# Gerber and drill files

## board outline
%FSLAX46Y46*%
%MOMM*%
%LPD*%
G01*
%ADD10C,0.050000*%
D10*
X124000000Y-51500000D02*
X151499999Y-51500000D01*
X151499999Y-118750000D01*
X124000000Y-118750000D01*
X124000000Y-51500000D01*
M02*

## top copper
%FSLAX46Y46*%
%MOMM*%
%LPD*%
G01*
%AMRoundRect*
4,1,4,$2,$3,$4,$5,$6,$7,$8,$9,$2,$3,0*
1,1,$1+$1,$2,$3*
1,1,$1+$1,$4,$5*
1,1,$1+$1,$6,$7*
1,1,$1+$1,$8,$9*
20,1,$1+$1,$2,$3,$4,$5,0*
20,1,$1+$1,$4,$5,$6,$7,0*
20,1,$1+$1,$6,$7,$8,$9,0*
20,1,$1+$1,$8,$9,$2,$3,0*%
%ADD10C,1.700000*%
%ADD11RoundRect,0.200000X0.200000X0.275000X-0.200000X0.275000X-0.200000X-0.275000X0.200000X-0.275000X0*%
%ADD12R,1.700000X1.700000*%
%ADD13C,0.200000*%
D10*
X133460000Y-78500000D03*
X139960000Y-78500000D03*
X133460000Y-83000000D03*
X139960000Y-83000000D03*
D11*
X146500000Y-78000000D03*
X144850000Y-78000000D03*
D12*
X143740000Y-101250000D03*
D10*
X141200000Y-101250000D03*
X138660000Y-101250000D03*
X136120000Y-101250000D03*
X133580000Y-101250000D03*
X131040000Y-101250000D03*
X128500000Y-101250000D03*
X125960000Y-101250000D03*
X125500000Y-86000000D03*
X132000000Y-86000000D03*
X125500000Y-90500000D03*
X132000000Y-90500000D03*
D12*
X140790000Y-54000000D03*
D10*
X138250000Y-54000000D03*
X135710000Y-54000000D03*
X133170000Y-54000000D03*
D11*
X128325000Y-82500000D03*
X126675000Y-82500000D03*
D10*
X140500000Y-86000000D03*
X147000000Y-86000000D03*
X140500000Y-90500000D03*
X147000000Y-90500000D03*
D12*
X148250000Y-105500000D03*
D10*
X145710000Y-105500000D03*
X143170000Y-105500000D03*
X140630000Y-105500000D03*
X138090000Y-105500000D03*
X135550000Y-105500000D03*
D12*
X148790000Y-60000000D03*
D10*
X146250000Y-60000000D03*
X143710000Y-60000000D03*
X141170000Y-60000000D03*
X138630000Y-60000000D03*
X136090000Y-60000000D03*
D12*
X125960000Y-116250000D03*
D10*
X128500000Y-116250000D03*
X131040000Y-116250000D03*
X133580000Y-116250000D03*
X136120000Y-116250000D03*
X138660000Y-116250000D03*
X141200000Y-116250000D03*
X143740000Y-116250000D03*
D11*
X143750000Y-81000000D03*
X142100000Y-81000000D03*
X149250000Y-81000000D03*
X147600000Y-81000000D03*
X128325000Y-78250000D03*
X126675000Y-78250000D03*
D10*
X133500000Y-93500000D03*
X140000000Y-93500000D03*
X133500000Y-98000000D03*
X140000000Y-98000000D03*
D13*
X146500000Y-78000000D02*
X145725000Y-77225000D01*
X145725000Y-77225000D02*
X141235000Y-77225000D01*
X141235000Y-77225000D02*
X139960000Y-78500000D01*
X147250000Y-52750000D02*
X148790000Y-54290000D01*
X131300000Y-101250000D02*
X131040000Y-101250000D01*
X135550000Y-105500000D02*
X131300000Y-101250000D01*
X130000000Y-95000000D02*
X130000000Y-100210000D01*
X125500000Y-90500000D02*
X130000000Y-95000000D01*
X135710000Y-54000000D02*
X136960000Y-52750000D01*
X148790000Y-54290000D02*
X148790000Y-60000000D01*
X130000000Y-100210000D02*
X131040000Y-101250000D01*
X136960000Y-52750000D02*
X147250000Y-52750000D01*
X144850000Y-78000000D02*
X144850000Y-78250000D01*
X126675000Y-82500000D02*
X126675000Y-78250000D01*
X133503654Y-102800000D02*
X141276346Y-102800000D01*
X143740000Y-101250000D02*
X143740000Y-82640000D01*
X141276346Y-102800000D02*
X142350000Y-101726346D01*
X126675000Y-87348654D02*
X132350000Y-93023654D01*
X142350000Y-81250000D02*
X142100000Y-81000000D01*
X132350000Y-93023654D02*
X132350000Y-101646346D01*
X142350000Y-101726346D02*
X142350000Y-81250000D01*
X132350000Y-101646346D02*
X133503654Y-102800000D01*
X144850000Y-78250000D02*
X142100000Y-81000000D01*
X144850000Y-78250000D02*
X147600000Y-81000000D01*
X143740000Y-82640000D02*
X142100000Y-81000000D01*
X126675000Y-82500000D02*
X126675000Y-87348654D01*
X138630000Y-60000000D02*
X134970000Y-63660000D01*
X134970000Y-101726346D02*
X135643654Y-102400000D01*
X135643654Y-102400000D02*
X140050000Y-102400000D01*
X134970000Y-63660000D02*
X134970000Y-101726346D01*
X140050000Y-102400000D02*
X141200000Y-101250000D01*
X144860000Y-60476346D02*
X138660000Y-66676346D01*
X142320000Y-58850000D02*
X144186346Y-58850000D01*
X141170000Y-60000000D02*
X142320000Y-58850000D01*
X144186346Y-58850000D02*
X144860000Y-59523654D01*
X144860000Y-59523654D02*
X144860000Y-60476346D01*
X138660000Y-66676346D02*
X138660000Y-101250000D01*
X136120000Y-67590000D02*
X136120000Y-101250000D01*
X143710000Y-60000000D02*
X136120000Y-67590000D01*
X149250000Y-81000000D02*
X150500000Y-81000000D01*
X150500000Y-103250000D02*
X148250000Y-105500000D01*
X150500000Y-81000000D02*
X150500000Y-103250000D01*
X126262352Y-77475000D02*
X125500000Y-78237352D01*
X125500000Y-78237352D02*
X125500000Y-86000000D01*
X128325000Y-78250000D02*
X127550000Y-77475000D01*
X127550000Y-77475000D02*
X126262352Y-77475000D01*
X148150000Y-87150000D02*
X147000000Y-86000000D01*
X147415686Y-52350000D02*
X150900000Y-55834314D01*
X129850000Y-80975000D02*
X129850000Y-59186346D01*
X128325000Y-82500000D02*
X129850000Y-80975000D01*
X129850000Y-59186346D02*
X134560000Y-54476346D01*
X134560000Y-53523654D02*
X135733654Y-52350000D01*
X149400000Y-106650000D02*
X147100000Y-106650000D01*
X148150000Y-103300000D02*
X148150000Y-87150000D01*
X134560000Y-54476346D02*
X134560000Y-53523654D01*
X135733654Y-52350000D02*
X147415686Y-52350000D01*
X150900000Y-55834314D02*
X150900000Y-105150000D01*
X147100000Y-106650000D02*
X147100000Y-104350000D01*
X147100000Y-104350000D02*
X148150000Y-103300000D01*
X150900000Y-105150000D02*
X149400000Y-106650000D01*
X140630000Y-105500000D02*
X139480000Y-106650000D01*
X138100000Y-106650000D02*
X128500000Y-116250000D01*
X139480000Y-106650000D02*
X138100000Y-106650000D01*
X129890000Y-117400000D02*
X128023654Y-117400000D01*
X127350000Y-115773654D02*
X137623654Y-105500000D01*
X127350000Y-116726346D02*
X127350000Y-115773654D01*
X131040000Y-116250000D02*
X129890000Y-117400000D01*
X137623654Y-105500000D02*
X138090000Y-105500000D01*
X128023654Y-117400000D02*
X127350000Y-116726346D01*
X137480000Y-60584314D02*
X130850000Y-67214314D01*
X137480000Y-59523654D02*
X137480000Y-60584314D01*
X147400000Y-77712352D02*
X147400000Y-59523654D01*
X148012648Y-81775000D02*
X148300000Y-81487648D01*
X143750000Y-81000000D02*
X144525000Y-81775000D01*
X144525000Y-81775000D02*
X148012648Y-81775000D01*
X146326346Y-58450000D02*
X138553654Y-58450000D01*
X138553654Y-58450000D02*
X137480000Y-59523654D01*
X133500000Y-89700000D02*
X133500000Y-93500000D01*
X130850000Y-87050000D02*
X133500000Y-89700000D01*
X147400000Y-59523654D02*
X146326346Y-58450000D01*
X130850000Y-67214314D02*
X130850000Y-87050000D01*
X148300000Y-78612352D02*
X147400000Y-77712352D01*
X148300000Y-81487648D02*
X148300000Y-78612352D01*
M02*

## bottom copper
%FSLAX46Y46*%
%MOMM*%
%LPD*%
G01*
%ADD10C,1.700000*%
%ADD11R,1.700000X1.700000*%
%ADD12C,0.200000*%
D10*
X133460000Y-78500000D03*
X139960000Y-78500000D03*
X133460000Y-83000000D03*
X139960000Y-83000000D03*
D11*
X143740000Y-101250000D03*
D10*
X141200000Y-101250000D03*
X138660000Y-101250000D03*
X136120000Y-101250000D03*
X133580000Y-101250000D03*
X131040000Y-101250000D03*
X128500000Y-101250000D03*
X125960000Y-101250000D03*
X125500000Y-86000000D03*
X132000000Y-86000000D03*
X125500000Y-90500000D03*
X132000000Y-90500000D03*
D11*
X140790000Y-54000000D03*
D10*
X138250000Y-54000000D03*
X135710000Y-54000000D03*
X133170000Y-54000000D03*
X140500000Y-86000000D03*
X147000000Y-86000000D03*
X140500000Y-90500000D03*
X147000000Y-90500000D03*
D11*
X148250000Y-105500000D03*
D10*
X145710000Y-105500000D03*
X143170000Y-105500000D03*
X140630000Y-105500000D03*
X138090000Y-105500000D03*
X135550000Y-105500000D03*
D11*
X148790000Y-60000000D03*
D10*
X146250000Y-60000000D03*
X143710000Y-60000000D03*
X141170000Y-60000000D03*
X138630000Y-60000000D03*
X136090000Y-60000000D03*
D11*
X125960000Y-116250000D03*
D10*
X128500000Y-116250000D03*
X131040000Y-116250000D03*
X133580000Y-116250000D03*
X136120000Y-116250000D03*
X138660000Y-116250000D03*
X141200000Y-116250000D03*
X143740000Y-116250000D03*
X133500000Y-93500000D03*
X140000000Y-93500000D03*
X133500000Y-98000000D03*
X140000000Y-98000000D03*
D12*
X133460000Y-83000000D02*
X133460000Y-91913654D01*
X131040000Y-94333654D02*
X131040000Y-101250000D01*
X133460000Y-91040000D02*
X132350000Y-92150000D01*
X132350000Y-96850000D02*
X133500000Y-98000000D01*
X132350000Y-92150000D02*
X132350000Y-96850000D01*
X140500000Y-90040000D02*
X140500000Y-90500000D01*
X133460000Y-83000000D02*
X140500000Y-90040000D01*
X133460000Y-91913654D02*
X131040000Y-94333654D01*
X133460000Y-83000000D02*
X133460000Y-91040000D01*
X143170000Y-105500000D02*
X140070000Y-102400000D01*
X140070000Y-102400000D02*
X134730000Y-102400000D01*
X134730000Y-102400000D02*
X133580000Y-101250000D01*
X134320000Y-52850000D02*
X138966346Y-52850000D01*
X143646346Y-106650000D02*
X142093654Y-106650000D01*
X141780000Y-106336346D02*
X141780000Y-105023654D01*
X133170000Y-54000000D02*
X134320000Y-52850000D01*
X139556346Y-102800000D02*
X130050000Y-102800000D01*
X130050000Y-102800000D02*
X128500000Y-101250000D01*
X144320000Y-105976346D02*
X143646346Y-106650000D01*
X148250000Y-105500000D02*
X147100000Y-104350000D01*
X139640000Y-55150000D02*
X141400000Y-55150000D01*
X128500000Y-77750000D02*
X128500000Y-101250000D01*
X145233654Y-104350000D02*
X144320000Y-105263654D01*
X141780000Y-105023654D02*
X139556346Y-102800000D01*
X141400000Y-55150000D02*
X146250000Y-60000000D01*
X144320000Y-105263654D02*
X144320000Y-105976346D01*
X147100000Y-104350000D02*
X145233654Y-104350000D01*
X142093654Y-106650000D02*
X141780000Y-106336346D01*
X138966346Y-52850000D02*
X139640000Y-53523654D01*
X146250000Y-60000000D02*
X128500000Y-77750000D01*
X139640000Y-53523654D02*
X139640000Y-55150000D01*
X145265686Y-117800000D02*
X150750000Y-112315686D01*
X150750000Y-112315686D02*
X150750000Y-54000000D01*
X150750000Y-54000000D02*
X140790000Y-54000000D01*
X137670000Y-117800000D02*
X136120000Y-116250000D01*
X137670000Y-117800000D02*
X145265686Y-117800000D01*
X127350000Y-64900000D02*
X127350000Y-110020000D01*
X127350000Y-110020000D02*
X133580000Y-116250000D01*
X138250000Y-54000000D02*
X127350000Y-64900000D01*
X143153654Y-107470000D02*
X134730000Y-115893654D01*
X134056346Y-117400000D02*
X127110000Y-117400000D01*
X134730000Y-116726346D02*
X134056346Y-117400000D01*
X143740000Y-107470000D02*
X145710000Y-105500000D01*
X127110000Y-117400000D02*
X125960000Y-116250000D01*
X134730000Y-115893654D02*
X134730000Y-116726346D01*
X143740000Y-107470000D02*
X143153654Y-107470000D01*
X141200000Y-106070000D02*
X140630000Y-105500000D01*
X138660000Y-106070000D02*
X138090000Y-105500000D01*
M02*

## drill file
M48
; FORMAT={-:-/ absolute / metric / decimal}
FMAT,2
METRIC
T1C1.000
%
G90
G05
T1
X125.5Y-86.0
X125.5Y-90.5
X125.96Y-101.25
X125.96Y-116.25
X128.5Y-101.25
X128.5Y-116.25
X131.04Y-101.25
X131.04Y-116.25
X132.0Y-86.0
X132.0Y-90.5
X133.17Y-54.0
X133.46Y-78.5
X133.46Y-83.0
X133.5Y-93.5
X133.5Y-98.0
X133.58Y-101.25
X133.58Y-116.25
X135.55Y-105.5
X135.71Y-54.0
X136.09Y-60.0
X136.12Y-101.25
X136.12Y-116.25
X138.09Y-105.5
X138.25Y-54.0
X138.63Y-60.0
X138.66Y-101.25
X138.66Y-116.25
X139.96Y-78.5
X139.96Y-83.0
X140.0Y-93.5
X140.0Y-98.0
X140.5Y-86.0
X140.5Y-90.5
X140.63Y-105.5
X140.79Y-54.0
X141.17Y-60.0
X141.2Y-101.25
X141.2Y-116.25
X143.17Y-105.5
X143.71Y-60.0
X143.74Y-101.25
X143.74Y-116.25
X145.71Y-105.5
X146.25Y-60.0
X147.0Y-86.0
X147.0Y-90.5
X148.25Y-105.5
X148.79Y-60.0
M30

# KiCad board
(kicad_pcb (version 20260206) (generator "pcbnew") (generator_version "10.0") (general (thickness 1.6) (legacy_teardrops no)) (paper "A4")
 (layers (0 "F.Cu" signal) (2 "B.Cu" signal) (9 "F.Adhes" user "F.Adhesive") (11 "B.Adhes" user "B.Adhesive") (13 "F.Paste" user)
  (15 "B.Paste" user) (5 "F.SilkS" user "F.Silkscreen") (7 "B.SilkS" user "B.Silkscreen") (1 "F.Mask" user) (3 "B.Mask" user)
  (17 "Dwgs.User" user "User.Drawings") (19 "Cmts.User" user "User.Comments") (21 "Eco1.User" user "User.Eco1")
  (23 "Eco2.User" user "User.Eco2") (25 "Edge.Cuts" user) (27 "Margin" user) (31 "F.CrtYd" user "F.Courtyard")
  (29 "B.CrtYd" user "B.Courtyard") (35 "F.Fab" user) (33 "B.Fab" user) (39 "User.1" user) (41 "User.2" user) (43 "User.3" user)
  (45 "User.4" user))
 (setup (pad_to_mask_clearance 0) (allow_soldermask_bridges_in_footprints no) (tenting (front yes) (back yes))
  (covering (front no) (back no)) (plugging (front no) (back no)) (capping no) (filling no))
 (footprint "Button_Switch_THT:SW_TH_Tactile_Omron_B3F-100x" (layer "F.Cu") (at 133.46 78.5)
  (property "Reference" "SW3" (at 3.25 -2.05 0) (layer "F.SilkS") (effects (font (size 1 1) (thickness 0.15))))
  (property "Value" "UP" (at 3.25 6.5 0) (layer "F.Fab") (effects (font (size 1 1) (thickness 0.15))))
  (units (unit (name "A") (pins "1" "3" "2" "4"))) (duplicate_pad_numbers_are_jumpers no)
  (pad "1" thru_hole circle (at 0 0) (size 1.7 1.7) (drill 1) (layers "*.Cu" "*.Mask") (remove_unused_layers no) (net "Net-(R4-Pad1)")
   (thermal_bridge_angle 90))
  (pad "1" thru_hole circle (at 6.5 0) (size 1.7 1.7) (drill 1) (layers "*.Cu" "*.Mask") (remove_unused_layers no) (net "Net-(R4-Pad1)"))
  (pad "2" thru_hole circle (at 0 4.5) (size 1.7 1.7) (drill 1) (layers "*.Cu" "*.Mask") (remove_unused_layers no) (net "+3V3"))
  (pad "2" thru_hole circle (at 6.5 4.5) (size 1.7 1.7) (drill 1) (layers "*.Cu" "*.Mask") (remove_unused_layers no)
   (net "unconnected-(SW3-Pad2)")))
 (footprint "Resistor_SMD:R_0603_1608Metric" (layer "F.Cu") (at 145.675 78 180)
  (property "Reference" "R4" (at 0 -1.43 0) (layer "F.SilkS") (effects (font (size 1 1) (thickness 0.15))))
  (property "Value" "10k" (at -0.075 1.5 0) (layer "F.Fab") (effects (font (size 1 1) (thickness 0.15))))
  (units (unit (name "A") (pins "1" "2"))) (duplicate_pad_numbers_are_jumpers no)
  (pad "1" smd roundrect (at -0.825 0 180) (size 0.8 0.95) (layers "F.Cu" "F.Mask" "F.Paste") (roundrect_rratio 0.25) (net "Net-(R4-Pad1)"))
  (pad "2" smd roundrect (at 0.825 0 180) (size 0.8 0.95) (layers "F.Cu" "F.Mask" "F.Paste") (roundrect_rratio 0.25) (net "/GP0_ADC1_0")))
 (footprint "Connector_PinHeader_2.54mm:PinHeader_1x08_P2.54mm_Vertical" (layer "F.Cu") (at 143.74 101.25 -90)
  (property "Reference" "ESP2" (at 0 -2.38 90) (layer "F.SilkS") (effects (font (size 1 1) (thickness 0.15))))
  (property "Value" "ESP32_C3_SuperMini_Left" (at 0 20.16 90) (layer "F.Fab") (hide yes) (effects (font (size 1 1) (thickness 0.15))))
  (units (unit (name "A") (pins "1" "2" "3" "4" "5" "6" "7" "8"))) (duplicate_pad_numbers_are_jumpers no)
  (pad "1" thru_hole rect (at 0 0 270) (size 1.7 1.7) (drill 1) (layers "*.Cu" "*.Mask") (remove_unused_layers no) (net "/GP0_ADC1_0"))
  (pad "2" thru_hole circle (at 0 2.54 270) (size 1.7 1.7) (drill 1) (layers "*.Cu" "*.Mask") (remove_unused_layers no) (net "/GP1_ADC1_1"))
  (pad "3" thru_hole circle (at 0 5.08 270) (size 1.7 1.7) (drill 1) (layers "*.Cu" "*.Mask") (remove_unused_layers no) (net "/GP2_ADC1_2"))
  (pad "4" thru_hole circle (at 0 7.62 270) (size 1.7 1.7) (drill 1) (layers "*.Cu" "*.Mask") (remove_unused_layers no) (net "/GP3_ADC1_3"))
  (pad "5" thru_hole circle (at 0 10.16 270) (size 1.7 1.7) (drill 1) (layers "*.Cu" "*.Mask") (remove_unused_layers no) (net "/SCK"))
  (pad "6" thru_hole circle (at 0 12.7 270) (size 1.7 1.7) (drill 1) (layers "*.Cu" "*.Mask") (remove_unused_layers no) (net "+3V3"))
  (pad "7" thru_hole circle (at 0 15.24 270) (size 1.7 1.7) (drill 1) (layers "*.Cu" "*.Mask") (remove_unused_layers no) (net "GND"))
  (pad "8" thru_hole circle (at 0 17.78 270) (size 1.7 1.7) (drill 1) (layers "*.Cu" "*.Mask") (remove_unused_layers no)
   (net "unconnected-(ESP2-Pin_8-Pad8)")))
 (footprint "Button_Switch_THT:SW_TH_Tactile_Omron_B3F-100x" (layer "F.Cu") (at 125.5 86)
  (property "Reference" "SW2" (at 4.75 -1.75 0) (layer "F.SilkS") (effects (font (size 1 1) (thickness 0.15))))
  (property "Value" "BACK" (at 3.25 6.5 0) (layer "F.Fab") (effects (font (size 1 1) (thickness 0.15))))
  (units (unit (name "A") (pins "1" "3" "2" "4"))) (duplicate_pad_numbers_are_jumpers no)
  (pad "1" thru_hole circle (at 0 0) (size 1.7 1.7) (drill 1) (layers "*.Cu" "*.Mask") (remove_unused_layers no) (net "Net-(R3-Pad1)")
   (thermal_bridge_angle 90))
  (pad "1" thru_hole circle (at 6.5 0) (size 1.7 1.7) (drill 1) (layers "*.Cu" "*.Mask") (remove_unused_layers no) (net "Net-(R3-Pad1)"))
  (pad "2" thru_hole circle (at 0 4.5) (size 1.7 1.7) (drill 1) (layers "*.Cu" "*.Mask") (remove_unused_layers no) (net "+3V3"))
  (pad "2" thru_hole circle (at 6.5 4.5) (size 1.7 1.7) (drill 1) (layers "*.Cu" "*.Mask") (remove_unused_layers no)
   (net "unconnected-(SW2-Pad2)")))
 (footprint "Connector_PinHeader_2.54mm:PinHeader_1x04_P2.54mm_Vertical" (layer "F.Cu") (at 140.79 54 -90)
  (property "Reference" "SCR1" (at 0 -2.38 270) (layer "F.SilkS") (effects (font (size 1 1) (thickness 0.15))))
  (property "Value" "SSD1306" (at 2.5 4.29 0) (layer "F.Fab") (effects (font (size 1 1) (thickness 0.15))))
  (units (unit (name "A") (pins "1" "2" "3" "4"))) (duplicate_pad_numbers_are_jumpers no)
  (pad "1" thru_hole rect (at 0 0 270) (size 1.7 1.7) (drill 1) (layers "*.Cu" "*.Mask") (remove_unused_layers no) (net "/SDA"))
  (pad "2" thru_hole circle (at 0 2.54 270) (size 1.7 1.7) (drill 1) (layers "*.Cu" "*.Mask") (remove_unused_layers no) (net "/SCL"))
  (pad "3" thru_hole circle (at 0 5.08 270) (size 1.7 1.7) (drill 1) (layers "*.Cu" "*.Mask") (remove_unused_layers no) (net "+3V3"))
  (pad "4" thru_hole circle (at 0 7.62 270) (size 1.7 1.7) (drill 1) (layers "*.Cu" "*.Mask") (remove_unused_layers no) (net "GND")))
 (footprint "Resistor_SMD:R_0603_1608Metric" (layer "F.Cu") (at 127.5 82.5 180)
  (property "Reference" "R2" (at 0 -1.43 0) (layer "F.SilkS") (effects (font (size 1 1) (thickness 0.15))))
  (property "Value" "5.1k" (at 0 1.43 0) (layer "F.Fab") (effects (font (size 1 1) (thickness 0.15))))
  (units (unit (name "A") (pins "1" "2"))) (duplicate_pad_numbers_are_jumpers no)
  (pad "1" smd roundrect (at -0.825 0 180) (size 0.8 0.95) (layers "F.Cu" "F.Mask" "F.Paste") (roundrect_rratio 0.25) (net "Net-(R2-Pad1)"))
  (pad "2" smd roundrect (at 0.825 0 180) (size 0.8 0.95) (layers "F.Cu" "F.Mask" "F.Paste") (roundrect_rratio 0.25) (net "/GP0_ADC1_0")))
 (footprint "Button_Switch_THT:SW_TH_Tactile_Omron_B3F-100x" (layer "F.Cu") (at 140.5 86)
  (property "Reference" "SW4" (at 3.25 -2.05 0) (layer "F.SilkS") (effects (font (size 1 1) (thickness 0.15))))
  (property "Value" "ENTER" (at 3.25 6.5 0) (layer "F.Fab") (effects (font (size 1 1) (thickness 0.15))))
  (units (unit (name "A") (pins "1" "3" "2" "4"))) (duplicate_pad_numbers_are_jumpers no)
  (pad "1" thru_hole circle (at 0 0) (size 1.7 1.7) (drill 1) (layers "*.Cu" "*.Mask") (remove_unused_layers no) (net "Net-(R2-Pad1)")
   (thermal_bridge_angle 90))
  (pad "1" thru_hole circle (at 6.5 0) (size 1.7 1.7) (drill 1) (layers "*.Cu" "*.Mask") (remove_unused_layers no) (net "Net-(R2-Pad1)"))
  (pad "2" thru_hole circle (at 0 4.5) (size 1.7 1.7) (drill 1) (layers "*.Cu" "*.Mask") (remove_unused_layers no) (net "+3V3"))
  (pad "2" thru_hole circle (at 6.5 4.5) (size 1.7 1.7) (drill 1) (layers "*.Cu" "*.Mask") (remove_unused_layers no)
   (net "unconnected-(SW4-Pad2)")))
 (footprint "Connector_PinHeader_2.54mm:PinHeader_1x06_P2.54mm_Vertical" (layer "F.Cu") (at 148.25 105.5 -90)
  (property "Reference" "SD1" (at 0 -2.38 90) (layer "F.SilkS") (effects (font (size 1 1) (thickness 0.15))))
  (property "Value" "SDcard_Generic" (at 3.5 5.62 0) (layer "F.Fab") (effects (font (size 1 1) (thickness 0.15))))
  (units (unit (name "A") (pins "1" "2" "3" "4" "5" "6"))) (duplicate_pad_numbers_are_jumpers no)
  (pad "1" thru_hole rect (at 0 0 270) (size 1.7 1.7) (drill 1) (layers "*.Cu" "*.Mask") (remove_unused_layers no) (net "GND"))
  (pad "2" thru_hole circle (at 0 2.54 270) (size 1.7 1.7) (drill 1) (layers "*.Cu" "*.Mask") (remove_unused_layers no) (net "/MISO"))
  (pad "3" thru_hole circle (at 0 5.08 270) (size 1.7 1.7) (drill 1) (layers "*.Cu" "*.Mask") (remove_unused_layers no) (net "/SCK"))
  (pad "4" thru_hole circle (at 0 7.62 270) (size 1.7 1.7) (drill 1) (layers "*.Cu" "*.Mask") (remove_unused_layers no) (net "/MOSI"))
  (pad "5" thru_hole circle (at 0 10.16 270) (size 1.7 1.7) (drill 1) (layers "*.Cu" "*.Mask") (remove_unused_layers no) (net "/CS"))
  (pad "6" thru_hole circle (at 0 12.7 270) (size 1.7 1.7) (drill 1) (layers "*.Cu" "*.Mask") (remove_unused_layers no) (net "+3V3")))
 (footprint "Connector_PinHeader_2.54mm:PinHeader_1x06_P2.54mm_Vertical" (layer "F.Cu") (at 148.79 60 -90)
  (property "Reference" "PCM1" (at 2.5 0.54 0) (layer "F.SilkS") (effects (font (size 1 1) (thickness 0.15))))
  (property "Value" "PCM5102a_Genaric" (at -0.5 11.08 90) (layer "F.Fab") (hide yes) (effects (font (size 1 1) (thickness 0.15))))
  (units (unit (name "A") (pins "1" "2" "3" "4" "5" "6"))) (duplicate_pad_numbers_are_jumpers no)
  (pad "1" thru_hole rect (at 0 0 270) (size 1.7 1.7) (drill 1) (layers "*.Cu" "*.Mask") (remove_unused_layers no) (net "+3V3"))
  (pad "2" thru_hole circle (at 0 2.54 270) (size 1.7 1.7) (drill 1) (layers "*.Cu" "*.Mask") (remove_unused_layers no) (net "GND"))
  (pad "3" thru_hole circle (at 0 5.08 270) (size 1.7 1.7) (drill 1) (layers "*.Cu" "*.Mask") (remove_unused_layers no) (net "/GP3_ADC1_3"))
  (pad "4" thru_hole circle (at 0 7.62 270) (size 1.7 1.7) (drill 1) (layers "*.Cu" "*.Mask") (remove_unused_layers no) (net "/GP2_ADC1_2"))
  (pad "5" thru_hole circle (at 0 10.16 270) (size 1.7 1.7) (drill 1) (layers "*.Cu" "*.Mask") (remove_unused_layers no) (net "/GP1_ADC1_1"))
  (pad "6" thru_hole circle (at 0 12.7 270) (size 1.7 1.7) (drill 1) (layers "*.Cu" "*.Mask") (remove_unused_layers no)
   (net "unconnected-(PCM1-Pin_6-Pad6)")))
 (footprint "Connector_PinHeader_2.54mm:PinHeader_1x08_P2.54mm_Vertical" (layer "F.Cu") (at 125.96 116.25 90)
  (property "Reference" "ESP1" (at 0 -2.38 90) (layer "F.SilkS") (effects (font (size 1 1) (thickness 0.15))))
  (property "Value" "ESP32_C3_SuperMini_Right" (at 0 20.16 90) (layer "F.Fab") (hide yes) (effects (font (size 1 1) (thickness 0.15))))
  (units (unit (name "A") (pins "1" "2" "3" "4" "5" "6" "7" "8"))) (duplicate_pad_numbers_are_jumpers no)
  (pad "1" thru_hole rect (at 0 0 90) (size 1.7 1.7) (drill 1) (layers "*.Cu" "*.Mask") (remove_unused_layers no) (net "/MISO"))
  (pad "2" thru_hole circle (at 0 2.54 90) (size 1.7 1.7) (drill 1) (layers "*.Cu" "*.Mask") (remove_unused_layers no) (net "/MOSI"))
  (pad "3" thru_hole circle (at 0 5.08 90) (size 1.7 1.7) (drill 1) (layers "*.Cu" "*.Mask") (remove_unused_layers no) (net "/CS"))
  (pad "4" thru_hole circle (at 0 7.62 90) (size 1.7 1.7) (drill 1) (layers "*.Cu" "*.Mask") (remove_unused_layers no) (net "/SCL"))
  (pad "5" thru_hole circle (at 0 10.16 90) (size 1.7 1.7) (drill 1) (layers "*.Cu" "*.Mask") (remove_unused_layers no) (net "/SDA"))
  (pad "6" thru_hole circle (at 0 12.7 90) (size 1.7 1.7) (drill 1) (layers "*.Cu" "*.Mask") (remove_unused_layers no)
   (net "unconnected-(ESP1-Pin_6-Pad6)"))
  (pad "7" thru_hole circle (at 0 15.24 90) (size 1.7 1.7) (drill 1) (layers "*.Cu" "*.Mask") (remove_unused_layers no)
   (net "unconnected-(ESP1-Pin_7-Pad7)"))
  (pad "8" thru_hole circle (at 0 17.78 90) (size 1.7 1.7) (drill 1) (layers "*.Cu" "*.Mask") (remove_unused_layers no)
   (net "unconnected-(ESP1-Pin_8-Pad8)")))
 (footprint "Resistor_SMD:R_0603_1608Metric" (layer "F.Cu") (at 142.925 81 180)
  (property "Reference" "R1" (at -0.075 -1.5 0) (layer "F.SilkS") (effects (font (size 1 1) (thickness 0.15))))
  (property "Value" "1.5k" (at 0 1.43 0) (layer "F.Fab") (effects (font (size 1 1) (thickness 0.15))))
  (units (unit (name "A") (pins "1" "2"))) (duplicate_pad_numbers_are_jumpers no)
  (pad "1" smd roundrect (at -0.825 0 180) (size 0.8 0.95) (layers "F.Cu" "F.Mask" "F.Paste") (roundrect_rratio 0.25) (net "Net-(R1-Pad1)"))
  (pad "2" smd roundrect (at 0.825 0 180) (size 0.8 0.95) (layers "F.Cu" "F.Mask" "F.Paste") (roundrect_rratio 0.25) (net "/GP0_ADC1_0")))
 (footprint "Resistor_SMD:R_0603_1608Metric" (layer "F.Cu") (at 148.425 81 180)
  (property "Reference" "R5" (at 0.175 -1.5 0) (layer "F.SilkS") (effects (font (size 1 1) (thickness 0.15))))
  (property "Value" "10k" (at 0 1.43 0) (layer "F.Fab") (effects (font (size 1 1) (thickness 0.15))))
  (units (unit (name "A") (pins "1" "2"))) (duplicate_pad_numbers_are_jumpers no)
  (pad "1" smd roundrect (at -0.825 0 180) (size 0.8 0.95) (layers "F.Cu" "F.Mask" "F.Paste") (roundrect_rratio 0.25) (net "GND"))
  (pad "2" smd roundrect (at 0.825 0 180) (size 0.8 0.95) (layers "F.Cu" "F.Mask" "F.Paste") (roundrect_rratio 0.25) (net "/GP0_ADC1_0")))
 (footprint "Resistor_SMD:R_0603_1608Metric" (layer "F.Cu") (at 127.5 78.25 180)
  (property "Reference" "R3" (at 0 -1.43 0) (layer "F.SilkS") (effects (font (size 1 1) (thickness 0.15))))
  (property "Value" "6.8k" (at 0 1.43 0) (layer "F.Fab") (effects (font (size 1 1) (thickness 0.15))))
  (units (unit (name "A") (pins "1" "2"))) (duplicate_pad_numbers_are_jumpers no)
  (pad "1" smd roundrect (at -0.825 0 180) (size 0.8 0.95) (layers "F.Cu" "F.Mask" "F.Paste") (roundrect_rratio 0.25) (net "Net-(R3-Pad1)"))
  (pad "2" smd roundrect (at 0.825 0 180) (size 0.8 0.95) (layers "F.Cu" "F.Mask" "F.Paste") (roundrect_rratio 0.25) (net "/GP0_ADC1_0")))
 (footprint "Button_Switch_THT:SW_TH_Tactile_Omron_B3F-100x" (layer "F.Cu") (at 133.5 93.5)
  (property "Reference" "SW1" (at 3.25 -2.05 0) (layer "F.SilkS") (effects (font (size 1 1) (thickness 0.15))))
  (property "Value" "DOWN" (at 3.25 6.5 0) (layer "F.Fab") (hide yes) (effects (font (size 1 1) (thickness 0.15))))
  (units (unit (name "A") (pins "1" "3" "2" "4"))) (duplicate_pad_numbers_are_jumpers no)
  (pad "1" thru_hole circle (at 0 0) (size 1.7 1.7) (drill 1) (layers "*.Cu" "*.Mask") (remove_unused_layers no) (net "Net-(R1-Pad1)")
   (thermal_bridge_angle 90))
  (pad "1" thru_hole circle (at 6.5 0) (size 1.7 1.7) (drill 1) (layers "*.Cu" "*.Mask") (remove_unused_layers no) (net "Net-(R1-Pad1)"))
  (pad "2" thru_hole circle (at 0 4.5) (size 1.7 1.7) (drill 1) (layers "*.Cu" "*.Mask") (remove_unused_layers no) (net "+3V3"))
  (pad "2" thru_hole circle (at 6.5 4.5) (size 1.7 1.7) (drill 1) (layers "*.Cu" "*.Mask") (remove_unused_layers no)
   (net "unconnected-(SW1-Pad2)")))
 (gr_rect (start 124 51.5) (end 151.499999 118.75) (stroke (width 0.05) (type default)) (fill no) (layer "Edge.Cuts"))
 (segment (start 146.5 78) (end 145.725 77.225) (width 0.2) (layer "F.Cu") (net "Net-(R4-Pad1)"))
 (segment (start 145.725 77.225) (end 141.235 77.225) (width 0.2) (layer "F.Cu") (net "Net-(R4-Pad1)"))
 (segment (start 141.235 77.225) (end 139.96 78.5) (width 0.2) (layer "F.Cu") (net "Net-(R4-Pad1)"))
 (segment (start 147.25 52.75) (end 148.79 54.29) (width 0.2) (layer "F.Cu") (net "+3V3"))
 (segment (start 131.3 101.25) (end 131.04 101.25) (width 0.2) (layer "F.Cu") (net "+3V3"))
 (segment (start 135.55 105.5) (end 131.3 101.25) (width 0.2) (layer "F.Cu") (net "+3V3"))
 (segment (start 130 95) (end 130 100.21) (width 0.2) (layer "F.Cu") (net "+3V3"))
 (segment (start 125.5 90.5) (end 130 95) (width 0.2) (layer "F.Cu") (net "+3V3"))
 (segment (start 135.71 54) (end 136.96 52.75) (width 0.2) (layer "F.Cu") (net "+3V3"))
 (segment (start 148.79 54.29) (end 148.79 60) (width 0.2) (layer "F.Cu") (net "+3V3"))
 (segment (start 130 100.21) (end 131.04 101.25) (width 0.2) (layer "F.Cu") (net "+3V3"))
 (segment (start 136.96 52.75) (end 147.25 52.75) (width 0.2) (layer "F.Cu") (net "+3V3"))
 (segment (start 133.46 83) (end 133.46 91.913654) (width 0.2) (layer "B.Cu") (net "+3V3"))
 (segment (start 131.04 94.333654) (end 131.04 101.25) (width 0.2) (layer "B.Cu") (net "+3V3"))
 (segment (start 133.46 91.04) (end 132.35 92.15) (width 0.2) (layer "B.Cu") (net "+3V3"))
 (segment (start 132.35 96.85) (end 133.5 98) (width 0.2) (layer "B.Cu") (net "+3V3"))
 (segment (start 132.35 92.15) (end 132.35 96.85) (width 0.2) (layer "B.Cu") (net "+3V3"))
 (segment (start 140.5 90.04) (end 140.5 90.5) (width 0.2) (layer "B.Cu") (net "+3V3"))
 (segment (start 133.46 83) (end 140.5 90.04) (width 0.2) (layer "B.Cu") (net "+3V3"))
 (segment (start 133.46 91.913654) (end 131.04 94.333654) (width 0.2) (layer "B.Cu") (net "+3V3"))
 (segment (start 133.46 83) (end 133.46 91.04) (width 0.2) (layer "B.Cu") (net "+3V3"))
 (segment (start 144.85 78) (end 144.85 78.25) (width 0.2) (layer "F.Cu") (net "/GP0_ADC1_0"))
 (segment (start 126.675 82.5) (end 126.675 78.25) (width 0.2) (layer "F.Cu") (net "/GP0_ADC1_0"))
 (segment (start 133.503654 102.8) (end 141.276346 102.8) (width 0.2) (layer "F.Cu") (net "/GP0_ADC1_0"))
 (segment (start 143.74 101.25) (end 143.74 82.64) (width 0.2) (layer "F.Cu") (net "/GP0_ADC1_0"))
 (segment (start 141.276346 102.8) (end 142.35 101.726346) (width 0.2) (layer "F.Cu") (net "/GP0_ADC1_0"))
 (segment (start 126.675 87.348654) (end 132.35 93.023654) (width 0.2) (layer "F.Cu") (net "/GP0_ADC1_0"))
 (segment (start 142.35 81.25) (end 142.1 81) (width 0.2) (layer "F.Cu") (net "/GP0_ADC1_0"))
 (segment (start 132.35 93.023654) (end 132.35 101.646346) (width 0.2) (layer "F.Cu") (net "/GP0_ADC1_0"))
 (segment (start 142.35 101.726346) (end 142.35 81.25) (width 0.2) (layer "F.Cu") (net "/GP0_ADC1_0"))
 (segment (start 132.35 101.646346) (end 133.503654 102.8) (width 0.2) (layer "F.Cu") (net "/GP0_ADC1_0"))
 (segment (start 144.85 78.25) (end 142.1 81) (width 0.2) (layer "F.Cu") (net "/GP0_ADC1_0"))
 (segment (start 144.85 78.25) (end 147.6 81) (width 0.2) (layer "F.Cu") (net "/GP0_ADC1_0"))
 (segment (start 143.74 82.64) (end 142.1 81) (width 0.2) (layer "F.Cu") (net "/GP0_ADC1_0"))
 (segment (start 126.675 82.5) (end 126.675 87.348654) (width 0.2) (layer "F.Cu") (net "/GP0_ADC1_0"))
 (segment (start 138.63 60) (end 134.97 63.66) (width 0.2) (layer "F.Cu") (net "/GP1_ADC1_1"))
 (segment (start 134.97 101.726346) (end 135.643654 102.4) (width 0.2) (layer "F.Cu") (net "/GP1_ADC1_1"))
 (segment (start 135.643654 102.4) (end 140.05 102.4) (width 0.2) (layer "F.Cu") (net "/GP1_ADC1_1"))
 (segment (start 134.97 63.66) (end 134.97 101.726346) (width 0.2) (layer "F.Cu") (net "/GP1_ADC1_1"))
 (segment (start 140.05 102.4) (end 141.2 101.25) (width 0.2) (layer "F.Cu") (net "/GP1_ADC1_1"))
 (segment (start 144.86 60.476346) (end 138.66 66.676346) (width 0.2) (layer "F.Cu") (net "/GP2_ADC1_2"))
 (segment (start 142.32 58.85) (end 144.186346 58.85) (width 0.2) (layer "F.Cu") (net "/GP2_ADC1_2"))
 (segment (start 141.17 60) (end 142.32 58.85) (width 0.2) (layer "F.Cu") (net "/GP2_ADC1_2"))
 (segment (start 144.186346 58.85) (end 144.86 59.523654) (width 0.2) (layer "F.Cu") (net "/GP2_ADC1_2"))
 (segment (start 144.86 59.523654) (end 144.86 60.476346) (width 0.2) (layer "F.Cu") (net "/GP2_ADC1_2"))
 (segment (start 138.66 66.676346) (end 138.66 101.25) (width 0.2) (layer "F.Cu") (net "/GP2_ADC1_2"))
 (segment (start 136.12 67.59) (end 136.12 101.25) (width 0.2) (layer "F.Cu") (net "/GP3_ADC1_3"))
 (segment (start 143.71 60) (end 136.12 67.59) (width 0.2) (layer "F.Cu") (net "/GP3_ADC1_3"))
 (segment (start 143.17 105.5) (end 140.07 102.4) (width 0.2) (layer "B.Cu") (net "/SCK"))
 (segment (start 140.07 102.4) (end 134.73 102.4) (width 0.2) (layer "B.Cu") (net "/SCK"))
 (segment (start 134.73 102.4) (end 133.58 101.25) (width 0.2) (layer "B.Cu") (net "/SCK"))
 (segment (start 149.25 81) (end 150.5 81) (width 0.2) (layer "F.Cu") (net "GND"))
 (segment (start 150.5 103.25) (end 148.25 105.5) (width 0.2) (layer "F.Cu") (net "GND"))
 (segment (start 150.5 81) (end 150.5 103.25) (width 0.2) (layer "F.Cu") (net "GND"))
 (segment (start 134.32 52.85) (end 138.966346 52.85) (width 0.2) (layer "B.Cu") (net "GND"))
 (segment (start 143.646346 106.65) (end 142.093654 106.65) (width 0.2) (layer "B.Cu") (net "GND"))
 (segment (start 141.78 106.336346) (end 141.78 105.023654) (width 0.2) (layer "B.Cu") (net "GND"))
 (segment (start 133.17 54) (end 134.32 52.85) (width 0.2) (layer "B.Cu") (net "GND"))
 (segment (start 139.556346 102.8) (end 130.05 102.8) (width 0.2) (layer "B.Cu") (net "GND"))
 (segment (start 130.05 102.8) (end 128.5 101.25) (width 0.2) (layer "B.Cu") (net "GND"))
 (segment (start 144.32 105.976346) (end 143.646346 106.65) (width 0.2) (layer "B.Cu") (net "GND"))
 (segment (start 148.25 105.5) (end 147.1 104.35) (width 0.2) (layer "B.Cu") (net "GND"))
 (segment (start 139.64 55.15) (end 141.4 55.15) (width 0.2) (layer "B.Cu") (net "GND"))
 (segment (start 128.5 77.75) (end 128.5 101.25) (width 0.2) (layer "B.Cu") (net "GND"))
 (segment (start 145.233654 104.35) (end 144.32 105.263654) (width 0.2) (layer "B.Cu") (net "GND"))
 (segment (start 141.78 105.023654) (end 139.556346 102.8) (width 0.2) (layer "B.Cu") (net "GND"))
 (segment (start 141.4 55.15) (end 146.25 60) (width 0.2) (layer "B.Cu") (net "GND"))
 (segment (start 144.32 105.263654) (end 144.32 105.976346) (width 0.2) (layer "B.Cu") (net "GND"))
 (segment (start 147.1 104.35) (end 145.233654 104.35) (width 0.2) (layer "B.Cu") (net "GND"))
 (segment (start 142.093654 106.65) (end 141.78 106.336346) (width 0.2) (layer "B.Cu") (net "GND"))
 (segment (start 138.966346 52.85) (end 139.64 53.523654) (width 0.2) (layer "B.Cu") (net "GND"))
 (segment (start 146.25 60) (end 128.5 77.75) (width 0.2) (layer "B.Cu") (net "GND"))
 (segment (start 139.64 53.523654) (end 139.64 55.15) (width 0.2) (layer "B.Cu") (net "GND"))
 (segment (start 126.262352 77.475) (end 125.5 78.237352) (width 0.2) (layer "F.Cu") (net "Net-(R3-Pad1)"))
 (segment (start 125.5 78.237352) (end 125.5 86) (width 0.2) (layer "F.Cu") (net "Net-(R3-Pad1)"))
 (segment (start 128.325 78.25) (end 127.55 77.475) (width 0.2) (layer "F.Cu") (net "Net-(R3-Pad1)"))
 (segment (start 127.55 77.475) (end 126.262352 77.475) (width 0.2) (layer "F.Cu") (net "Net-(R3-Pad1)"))
 (segment (start 145.265686 117.8) (end 150.75 112.315686) (width 0.2) (layer "B.Cu") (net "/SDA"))
 (segment (start 150.75 112.315686) (end 150.75 54) (width 0.2) (layer "B.Cu") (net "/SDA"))
 (segment (start 150.75 54) (end 140.79 54) (width 0.2) (layer "B.Cu") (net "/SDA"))
 (segment (start 137.67 117.8) (end 136.12 116.25) (width 0.2) (layer "B.Cu") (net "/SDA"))
 (segment (start 137.67 117.8) (end 145.265686 117.8) (width 0.2) (layer "B.Cu") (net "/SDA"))
 (segment (start 127.35 64.9) (end 127.35 110.02) (width 0.2) (layer "B.Cu") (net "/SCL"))
 (segment (start 127.35 110.02) (end 133.58 116.25) (width 0.2) (layer "B.Cu") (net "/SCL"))
 (segment (start 138.25 54) (end 127.35 64.9) (width 0.2) (layer "B.Cu") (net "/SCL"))
 (segment (start 148.15 87.15) (end 147 86) (width 0.2) (layer "F.Cu") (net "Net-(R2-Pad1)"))
 (segment (start 147.415686 52.35) (end 150.9 55.834314) (width 0.2) (layer "F.Cu") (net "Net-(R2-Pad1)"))
 (segment (start 129.85 80.975) (end 129.85 59.186346) (width 0.2) (layer "F.Cu") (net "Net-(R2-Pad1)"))
 (segment (start 128.325 82.5) (end 129.85 80.975) (width 0.2) (layer "F.Cu") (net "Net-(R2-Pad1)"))
 (segment (start 129.85 59.186346) (end 134.56 54.476346) (width 0.2) (layer "F.Cu") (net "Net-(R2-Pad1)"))
 (segment (start 134.56 53.523654) (end 135.733654 52.35) (width 0.2) (layer "F.Cu") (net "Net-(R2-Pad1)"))
 (segment (start 149.4 106.65) (end 147.1 106.65) (width 0.2) (layer "F.Cu") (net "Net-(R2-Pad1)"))
 (segment (start 148.15 103.3) (end 148.15 87.15) (width 0.2) (layer "F.Cu") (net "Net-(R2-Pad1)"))
 (segment (start 134.56 54.476346) (end 134.56 53.523654) (width 0.2) (layer "F.Cu") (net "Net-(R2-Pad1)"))
 (segment (start 135.733654 52.35) (end 147.415686 52.35) (width 0.2) (layer "F.Cu") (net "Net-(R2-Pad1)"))
 (segment (start 150.9 55.834314) (end 150.9 105.15) (width 0.2) (layer "F.Cu") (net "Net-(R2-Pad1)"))
 (segment (start 147.1 106.65) (end 147.1 104.35) (width 0.2) (layer "F.Cu") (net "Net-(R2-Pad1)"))
 (segment (start 147.1 104.35) (end 148.15 103.3) (width 0.2) (layer "F.Cu") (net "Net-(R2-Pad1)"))
 (segment (start 150.9 105.15) (end 149.4 106.65) (width 0.2) (layer "F.Cu") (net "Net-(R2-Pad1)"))
 (segment (start 143.153654 107.47) (end 134.73 115.893654) (width 0.2) (layer "B.Cu") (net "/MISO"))
 (segment (start 134.056346 117.4) (end 127.11 117.4) (width 0.2) (layer "B.Cu") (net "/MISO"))
 (segment (start 134.73 116.726346) (end 134.056346 117.4) (width 0.2) (layer "B.Cu") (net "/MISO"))
 (segment (start 143.74 107.47) (end 145.71 105.5) (width 0.2) (layer "B.Cu") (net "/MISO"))
 (segment (start 127.11 117.4) (end 125.96 116.25) (width 0.2) (layer "B.Cu") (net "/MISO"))
 (segment (start 134.73 115.893654) (end 134.73 116.726346) (width 0.2) (layer "B.Cu") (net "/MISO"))
 (segment (start 143.74 107.47) (end 143.153654 107.47) (width 0.2) (layer "B.Cu") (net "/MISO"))
 (segment (start 140.63 105.5) (end 139.48 106.65) (width 0.2) (layer "F.Cu") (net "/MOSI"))
 (segment (start 138.1 106.65) (end 128.5 116.25) (width 0.2) (layer "F.Cu") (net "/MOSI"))
 (segment (start 139.48 106.65) (end 138.1 106.65) (width 0.2) (layer "F.Cu") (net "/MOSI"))
 (segment (start 141.2 106.07) (end 140.63 105.5) (width 0.2) (layer "B.Cu") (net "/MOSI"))
 (segment (start 129.89 117.4) (end 128.023654 117.4) (width 0.2) (layer "F.Cu") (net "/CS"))
 (segment (start 127.35 115.773654) (end 137.623654 105.5) (width 0.2) (layer "F.Cu") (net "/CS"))
 (segment (start 127.35 116.726346) (end 127.35 115.773654) (width 0.2) (layer "F.Cu") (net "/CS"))
 (segment (start 131.04 116.25) (end 129.89 117.4) (width 0.2) (layer "F.Cu") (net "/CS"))
 (segment (start 137.623654 105.5) (end 138.09 105.5) (width 0.2) (layer "F.Cu") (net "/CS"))
 (segment (start 128.023654 117.4) (end 127.35 116.726346) (width 0.2) (layer "F.Cu") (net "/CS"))
 (segment (start 138.66 106.07) (end 138.09 105.5) (width 0.2) (layer "B.Cu") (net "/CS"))
 (segment (start 137.48 60.584314) (end 130.85 67.214314) (width 0.2) (layer "F.Cu") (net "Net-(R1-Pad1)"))
 (segment (start 137.48 59.523654) (end 137.48 60.584314) (width 0.2) (layer "F.Cu") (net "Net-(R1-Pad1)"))
 (segment (start 147.4 77.712352) (end 147.4 59.523654) (width 0.2) (layer "F.Cu") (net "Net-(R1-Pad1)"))
 (segment (start 148.012648 81.775) (end 148.3 81.487648) (width 0.2) (layer "F.Cu") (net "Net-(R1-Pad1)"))
 (segment (start 143.75 81) (end 144.525 81.775) (width 0.2) (layer "F.Cu") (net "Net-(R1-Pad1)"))
 (segment (start 144.525 81.775) (end 148.012648 81.775) (width 0.2) (layer "F.Cu") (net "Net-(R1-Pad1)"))
 (segment (start 146.326346 58.45) (end 138.553654 58.45) (width 0.2) (layer "F.Cu") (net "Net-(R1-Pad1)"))
 (segment (start 138.553654 58.45) (end 137.48 59.523654) (width 0.2) (layer "F.Cu") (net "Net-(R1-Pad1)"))
 (segment (start 133.5 89.7) (end 133.5 93.5) (width 0.2) (layer "F.Cu") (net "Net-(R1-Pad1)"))
 (segment (start 130.85 87.05) (end 133.5 89.7) (width 0.2) (layer "F.Cu") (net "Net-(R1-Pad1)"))
 (segment (start 147.4 59.523654) (end 146.326346 58.45) (width 0.2) (layer "F.Cu") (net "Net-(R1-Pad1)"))
 (segment (start 130.85 67.214314) (end 130.85 87.05) (width 0.2) (layer "F.Cu") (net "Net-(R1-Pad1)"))
 (segment (start 148.3 78.612352) (end 147.4 77.712352) (width 0.2) (layer "F.Cu") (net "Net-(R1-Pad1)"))
 (segment (start 148.3 81.487648) (end 148.3 78.612352) (width 0.2) (layer "F.Cu") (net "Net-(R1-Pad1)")))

